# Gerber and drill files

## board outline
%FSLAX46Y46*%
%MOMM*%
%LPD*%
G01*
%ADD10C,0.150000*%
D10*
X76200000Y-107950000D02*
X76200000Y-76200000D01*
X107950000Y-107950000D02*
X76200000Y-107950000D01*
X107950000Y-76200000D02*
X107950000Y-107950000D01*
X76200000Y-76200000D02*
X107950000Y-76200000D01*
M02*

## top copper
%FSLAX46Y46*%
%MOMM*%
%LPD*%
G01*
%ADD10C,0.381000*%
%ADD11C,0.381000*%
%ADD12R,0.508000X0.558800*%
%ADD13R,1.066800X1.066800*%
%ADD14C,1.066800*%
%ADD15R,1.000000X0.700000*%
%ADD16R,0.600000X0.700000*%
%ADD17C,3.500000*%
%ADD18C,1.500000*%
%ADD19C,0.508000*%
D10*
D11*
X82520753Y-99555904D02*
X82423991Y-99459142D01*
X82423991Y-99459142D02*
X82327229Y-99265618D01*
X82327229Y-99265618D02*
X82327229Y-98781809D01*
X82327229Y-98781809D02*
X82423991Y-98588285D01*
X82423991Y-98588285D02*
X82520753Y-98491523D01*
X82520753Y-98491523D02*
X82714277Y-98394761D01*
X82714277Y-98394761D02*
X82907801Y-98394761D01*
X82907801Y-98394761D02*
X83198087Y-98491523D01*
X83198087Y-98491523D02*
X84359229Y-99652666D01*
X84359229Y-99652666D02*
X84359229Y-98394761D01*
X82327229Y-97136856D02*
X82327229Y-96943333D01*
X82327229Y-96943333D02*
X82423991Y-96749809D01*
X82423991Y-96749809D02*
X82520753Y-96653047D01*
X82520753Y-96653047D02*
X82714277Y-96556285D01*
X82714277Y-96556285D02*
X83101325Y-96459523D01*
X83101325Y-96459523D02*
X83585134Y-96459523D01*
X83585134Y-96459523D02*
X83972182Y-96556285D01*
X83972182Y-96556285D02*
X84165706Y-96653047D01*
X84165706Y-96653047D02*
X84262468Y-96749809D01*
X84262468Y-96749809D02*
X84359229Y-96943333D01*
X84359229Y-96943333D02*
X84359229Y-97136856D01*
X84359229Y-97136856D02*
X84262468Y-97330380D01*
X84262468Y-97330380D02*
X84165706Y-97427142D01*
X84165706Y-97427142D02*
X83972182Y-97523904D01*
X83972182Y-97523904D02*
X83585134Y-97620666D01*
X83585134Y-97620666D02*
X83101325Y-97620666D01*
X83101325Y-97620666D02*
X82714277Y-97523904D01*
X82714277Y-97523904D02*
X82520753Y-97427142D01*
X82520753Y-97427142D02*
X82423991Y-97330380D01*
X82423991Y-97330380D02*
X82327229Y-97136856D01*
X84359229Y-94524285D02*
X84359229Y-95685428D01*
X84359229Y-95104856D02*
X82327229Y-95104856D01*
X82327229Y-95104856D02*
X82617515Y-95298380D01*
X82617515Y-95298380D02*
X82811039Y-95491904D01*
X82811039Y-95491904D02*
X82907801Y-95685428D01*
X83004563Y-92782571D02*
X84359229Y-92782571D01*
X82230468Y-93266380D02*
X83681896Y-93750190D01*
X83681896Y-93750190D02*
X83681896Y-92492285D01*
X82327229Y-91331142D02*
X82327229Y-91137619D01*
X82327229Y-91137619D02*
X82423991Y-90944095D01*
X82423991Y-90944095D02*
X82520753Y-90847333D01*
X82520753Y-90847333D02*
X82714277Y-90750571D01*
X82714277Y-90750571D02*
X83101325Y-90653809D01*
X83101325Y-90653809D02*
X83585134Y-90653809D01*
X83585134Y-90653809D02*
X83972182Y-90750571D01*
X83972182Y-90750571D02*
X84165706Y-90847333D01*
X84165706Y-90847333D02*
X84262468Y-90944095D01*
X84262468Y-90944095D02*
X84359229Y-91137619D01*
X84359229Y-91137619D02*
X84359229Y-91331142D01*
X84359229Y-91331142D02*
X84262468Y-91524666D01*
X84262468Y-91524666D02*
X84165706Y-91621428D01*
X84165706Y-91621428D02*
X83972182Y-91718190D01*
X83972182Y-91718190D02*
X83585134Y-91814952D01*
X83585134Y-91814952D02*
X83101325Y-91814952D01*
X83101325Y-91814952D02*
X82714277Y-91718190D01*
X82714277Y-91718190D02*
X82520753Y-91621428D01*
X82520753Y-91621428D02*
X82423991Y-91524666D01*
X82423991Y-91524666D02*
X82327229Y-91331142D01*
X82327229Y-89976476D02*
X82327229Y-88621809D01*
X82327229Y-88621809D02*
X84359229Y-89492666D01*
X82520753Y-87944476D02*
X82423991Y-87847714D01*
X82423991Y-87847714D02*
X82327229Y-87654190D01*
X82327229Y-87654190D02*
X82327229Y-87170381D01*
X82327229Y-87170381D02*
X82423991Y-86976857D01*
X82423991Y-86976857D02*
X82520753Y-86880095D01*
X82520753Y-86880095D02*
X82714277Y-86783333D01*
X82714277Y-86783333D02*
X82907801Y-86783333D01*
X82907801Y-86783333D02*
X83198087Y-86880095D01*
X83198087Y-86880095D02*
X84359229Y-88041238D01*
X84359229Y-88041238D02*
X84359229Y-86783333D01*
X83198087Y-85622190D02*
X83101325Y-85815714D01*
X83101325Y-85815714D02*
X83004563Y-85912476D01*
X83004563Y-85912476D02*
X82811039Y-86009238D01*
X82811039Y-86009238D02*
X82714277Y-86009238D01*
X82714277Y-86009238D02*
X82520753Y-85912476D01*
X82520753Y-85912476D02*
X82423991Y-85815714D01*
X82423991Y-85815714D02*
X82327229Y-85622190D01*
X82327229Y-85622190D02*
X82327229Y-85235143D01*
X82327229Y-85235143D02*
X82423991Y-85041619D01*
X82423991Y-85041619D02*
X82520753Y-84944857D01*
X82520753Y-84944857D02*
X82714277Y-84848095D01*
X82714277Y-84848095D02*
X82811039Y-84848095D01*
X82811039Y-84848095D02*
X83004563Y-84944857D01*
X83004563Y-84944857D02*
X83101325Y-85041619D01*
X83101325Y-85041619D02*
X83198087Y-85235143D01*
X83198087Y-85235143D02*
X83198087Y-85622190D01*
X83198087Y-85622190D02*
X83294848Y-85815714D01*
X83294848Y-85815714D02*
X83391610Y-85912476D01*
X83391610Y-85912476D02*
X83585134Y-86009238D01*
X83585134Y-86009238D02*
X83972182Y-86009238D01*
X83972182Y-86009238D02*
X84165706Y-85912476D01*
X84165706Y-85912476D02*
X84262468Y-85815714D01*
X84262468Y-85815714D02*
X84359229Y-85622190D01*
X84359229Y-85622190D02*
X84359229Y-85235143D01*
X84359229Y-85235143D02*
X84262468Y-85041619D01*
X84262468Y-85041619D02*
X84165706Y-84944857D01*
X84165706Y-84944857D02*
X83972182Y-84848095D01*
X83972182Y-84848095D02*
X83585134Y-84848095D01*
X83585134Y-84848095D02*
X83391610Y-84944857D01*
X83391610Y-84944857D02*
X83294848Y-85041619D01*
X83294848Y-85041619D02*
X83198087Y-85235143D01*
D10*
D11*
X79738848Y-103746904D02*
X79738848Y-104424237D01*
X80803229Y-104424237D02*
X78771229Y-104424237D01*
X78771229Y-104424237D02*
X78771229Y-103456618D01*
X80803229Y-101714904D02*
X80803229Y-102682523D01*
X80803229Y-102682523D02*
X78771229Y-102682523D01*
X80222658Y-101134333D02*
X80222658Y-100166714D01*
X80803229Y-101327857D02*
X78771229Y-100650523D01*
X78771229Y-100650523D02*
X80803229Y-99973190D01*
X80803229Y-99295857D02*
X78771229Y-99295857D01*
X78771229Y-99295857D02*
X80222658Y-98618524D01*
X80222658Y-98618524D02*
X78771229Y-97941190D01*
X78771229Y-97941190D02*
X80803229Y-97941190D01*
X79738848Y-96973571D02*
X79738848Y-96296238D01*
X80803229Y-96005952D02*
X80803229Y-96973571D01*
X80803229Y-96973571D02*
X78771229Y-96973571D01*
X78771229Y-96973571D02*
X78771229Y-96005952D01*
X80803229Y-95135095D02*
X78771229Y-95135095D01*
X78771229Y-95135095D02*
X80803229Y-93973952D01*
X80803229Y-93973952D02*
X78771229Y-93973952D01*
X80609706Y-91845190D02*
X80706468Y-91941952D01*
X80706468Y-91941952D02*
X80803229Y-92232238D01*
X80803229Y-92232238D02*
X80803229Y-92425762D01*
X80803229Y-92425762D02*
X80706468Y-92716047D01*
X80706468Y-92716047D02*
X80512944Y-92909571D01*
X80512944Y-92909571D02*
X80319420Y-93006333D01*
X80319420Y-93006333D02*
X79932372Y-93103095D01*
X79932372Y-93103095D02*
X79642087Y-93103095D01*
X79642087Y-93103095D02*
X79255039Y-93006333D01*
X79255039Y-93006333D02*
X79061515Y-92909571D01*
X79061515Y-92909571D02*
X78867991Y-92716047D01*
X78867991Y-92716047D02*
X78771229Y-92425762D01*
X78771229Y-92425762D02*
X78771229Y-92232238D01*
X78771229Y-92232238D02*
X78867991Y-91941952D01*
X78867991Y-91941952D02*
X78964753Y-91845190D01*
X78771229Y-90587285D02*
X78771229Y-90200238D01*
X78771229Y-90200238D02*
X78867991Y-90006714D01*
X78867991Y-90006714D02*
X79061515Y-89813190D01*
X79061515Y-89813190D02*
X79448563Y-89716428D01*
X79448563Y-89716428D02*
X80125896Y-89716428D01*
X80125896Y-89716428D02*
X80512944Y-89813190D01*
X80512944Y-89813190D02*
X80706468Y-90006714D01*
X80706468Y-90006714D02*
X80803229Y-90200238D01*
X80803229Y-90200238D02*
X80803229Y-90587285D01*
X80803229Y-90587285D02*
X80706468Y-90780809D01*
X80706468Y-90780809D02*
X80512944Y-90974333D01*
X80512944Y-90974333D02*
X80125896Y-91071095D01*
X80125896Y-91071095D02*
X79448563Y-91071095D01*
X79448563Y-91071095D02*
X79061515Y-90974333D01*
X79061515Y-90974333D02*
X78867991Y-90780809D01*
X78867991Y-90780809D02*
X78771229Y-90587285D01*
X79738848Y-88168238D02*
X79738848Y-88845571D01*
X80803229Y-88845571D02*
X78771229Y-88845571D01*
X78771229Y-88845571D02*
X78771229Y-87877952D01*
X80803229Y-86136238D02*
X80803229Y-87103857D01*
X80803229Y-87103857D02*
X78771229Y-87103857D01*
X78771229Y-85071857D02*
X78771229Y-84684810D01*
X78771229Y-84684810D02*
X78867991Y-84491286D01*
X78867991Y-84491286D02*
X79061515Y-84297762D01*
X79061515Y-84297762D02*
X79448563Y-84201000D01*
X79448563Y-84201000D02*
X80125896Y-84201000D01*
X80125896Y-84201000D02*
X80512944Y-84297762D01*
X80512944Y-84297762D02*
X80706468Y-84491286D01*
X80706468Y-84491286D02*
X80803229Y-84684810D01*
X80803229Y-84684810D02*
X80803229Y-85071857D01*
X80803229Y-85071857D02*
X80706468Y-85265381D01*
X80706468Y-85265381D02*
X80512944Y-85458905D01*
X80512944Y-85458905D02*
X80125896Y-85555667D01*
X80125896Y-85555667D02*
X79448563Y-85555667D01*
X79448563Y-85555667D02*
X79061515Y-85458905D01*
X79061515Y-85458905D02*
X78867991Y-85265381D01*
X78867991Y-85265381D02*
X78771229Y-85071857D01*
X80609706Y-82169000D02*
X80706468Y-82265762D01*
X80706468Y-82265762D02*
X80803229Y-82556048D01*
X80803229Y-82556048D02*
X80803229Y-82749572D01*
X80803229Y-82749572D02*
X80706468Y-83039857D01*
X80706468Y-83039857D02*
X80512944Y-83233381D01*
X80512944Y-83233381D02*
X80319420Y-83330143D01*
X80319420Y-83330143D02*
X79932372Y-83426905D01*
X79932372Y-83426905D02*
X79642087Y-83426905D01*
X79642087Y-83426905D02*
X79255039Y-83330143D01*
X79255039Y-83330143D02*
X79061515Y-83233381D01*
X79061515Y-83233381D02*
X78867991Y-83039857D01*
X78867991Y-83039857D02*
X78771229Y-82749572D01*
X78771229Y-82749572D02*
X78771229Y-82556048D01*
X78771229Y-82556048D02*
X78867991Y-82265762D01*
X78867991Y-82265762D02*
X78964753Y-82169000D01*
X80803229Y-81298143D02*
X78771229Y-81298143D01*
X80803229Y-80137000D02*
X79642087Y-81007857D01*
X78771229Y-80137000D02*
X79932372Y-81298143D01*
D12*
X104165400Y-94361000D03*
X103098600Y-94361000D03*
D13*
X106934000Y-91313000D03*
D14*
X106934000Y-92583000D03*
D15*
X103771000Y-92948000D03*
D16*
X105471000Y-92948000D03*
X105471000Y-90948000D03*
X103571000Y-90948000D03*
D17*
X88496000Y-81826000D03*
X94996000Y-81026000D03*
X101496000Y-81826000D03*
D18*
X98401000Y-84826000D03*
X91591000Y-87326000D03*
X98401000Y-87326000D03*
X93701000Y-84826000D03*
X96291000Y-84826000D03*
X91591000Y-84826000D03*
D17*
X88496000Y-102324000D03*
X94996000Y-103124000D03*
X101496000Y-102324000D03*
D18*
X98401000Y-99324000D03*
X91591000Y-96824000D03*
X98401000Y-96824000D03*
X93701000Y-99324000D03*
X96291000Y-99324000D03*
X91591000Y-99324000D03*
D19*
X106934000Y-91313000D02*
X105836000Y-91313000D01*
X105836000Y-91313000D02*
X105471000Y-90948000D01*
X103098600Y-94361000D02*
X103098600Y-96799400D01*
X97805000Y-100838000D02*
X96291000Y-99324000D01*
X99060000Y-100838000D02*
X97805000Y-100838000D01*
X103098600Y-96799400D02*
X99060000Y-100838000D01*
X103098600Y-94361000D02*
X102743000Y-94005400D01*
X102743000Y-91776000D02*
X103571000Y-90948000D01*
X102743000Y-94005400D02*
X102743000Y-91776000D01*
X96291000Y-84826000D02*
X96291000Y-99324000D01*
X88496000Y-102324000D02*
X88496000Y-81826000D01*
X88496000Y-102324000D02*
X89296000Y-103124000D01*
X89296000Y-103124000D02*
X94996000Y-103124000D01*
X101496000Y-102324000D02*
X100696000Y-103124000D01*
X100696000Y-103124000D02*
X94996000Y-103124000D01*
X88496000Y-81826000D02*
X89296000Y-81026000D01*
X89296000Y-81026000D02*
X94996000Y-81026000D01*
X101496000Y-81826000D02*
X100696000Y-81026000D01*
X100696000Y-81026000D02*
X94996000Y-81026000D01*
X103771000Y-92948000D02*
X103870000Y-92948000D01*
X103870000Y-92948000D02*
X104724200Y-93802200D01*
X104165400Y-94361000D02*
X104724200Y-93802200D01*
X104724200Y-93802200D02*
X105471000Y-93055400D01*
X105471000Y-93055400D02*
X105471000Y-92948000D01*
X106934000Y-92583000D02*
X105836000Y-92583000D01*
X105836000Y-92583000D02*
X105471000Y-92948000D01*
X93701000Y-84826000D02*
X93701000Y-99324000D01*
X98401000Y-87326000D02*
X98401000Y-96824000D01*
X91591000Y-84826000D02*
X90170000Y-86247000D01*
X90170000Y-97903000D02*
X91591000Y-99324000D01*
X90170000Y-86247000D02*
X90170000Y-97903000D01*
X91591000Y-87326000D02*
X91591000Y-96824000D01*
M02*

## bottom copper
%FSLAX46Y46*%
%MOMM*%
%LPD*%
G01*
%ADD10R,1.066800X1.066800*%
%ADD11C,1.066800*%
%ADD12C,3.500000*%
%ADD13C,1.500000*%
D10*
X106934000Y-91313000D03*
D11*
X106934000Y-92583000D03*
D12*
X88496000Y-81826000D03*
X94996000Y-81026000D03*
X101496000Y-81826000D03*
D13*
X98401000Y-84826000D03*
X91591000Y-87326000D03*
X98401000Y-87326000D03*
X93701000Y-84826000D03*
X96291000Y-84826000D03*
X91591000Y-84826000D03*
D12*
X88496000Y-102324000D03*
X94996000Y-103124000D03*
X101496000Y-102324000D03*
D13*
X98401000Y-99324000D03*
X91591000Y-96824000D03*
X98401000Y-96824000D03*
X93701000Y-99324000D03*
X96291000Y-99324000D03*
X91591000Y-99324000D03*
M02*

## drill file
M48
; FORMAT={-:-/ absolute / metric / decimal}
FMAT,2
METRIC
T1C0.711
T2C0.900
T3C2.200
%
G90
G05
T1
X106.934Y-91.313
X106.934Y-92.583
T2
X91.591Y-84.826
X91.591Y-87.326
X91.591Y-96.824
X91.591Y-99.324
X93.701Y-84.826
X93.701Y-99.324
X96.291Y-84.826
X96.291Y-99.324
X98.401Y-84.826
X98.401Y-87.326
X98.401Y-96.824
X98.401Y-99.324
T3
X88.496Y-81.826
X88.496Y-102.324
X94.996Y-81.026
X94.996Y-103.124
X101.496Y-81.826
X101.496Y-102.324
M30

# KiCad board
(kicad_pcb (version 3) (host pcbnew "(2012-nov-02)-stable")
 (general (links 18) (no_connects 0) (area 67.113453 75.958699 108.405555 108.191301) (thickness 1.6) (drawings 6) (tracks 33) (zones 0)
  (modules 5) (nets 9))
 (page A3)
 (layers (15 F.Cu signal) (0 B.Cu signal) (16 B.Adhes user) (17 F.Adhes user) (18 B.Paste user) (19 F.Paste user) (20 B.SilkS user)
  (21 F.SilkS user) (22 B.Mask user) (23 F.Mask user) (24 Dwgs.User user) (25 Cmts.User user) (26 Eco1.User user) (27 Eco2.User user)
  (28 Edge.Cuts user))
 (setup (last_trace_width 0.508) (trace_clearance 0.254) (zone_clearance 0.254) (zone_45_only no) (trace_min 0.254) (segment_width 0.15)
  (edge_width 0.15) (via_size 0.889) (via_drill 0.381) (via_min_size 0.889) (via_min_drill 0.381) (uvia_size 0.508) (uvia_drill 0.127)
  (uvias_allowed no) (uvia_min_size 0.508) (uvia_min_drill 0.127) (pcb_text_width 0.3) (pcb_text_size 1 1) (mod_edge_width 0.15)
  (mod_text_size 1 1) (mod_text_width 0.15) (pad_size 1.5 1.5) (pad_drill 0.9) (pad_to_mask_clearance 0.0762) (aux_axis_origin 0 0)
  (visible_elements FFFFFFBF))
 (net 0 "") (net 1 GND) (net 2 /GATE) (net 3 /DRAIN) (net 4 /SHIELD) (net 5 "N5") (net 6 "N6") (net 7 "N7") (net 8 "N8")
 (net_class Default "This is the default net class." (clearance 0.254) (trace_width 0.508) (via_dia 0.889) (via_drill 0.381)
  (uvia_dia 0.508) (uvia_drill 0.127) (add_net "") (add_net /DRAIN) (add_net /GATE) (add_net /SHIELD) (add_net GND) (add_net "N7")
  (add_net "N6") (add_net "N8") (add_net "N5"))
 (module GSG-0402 (layer F.Cu) (at 103.632 94.361) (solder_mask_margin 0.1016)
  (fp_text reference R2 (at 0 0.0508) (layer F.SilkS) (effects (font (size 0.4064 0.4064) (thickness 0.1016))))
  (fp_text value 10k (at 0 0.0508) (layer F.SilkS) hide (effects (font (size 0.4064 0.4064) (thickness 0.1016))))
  (pad 2 smd rect (at 0.5334 0) (size 0.508 0.5588) (layers F.Cu F.Paste F.Mask) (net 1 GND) (solder_mask_margin 0.1016))
  (pad 1 smd rect (at -0.5334 0) (size 0.508 0.5588) (layers F.Cu F.Paste F.Mask) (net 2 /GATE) (die_length -2147.483648)
   (solder_mask_margin 0.1016)))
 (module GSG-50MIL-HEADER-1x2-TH (layer F.Cu) (at 106.934 91.948 270)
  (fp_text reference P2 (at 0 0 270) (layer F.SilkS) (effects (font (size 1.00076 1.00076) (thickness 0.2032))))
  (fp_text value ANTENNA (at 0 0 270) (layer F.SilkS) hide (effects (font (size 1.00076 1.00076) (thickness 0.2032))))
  (pad 1 thru_hole rect (at -0.635 0 270) (size 1.0668 1.0668) (drill 0.7112) (layers *.Cu *.Mask) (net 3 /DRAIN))
  (pad 2 thru_hole circle (at 0.635 0 270) (size 1.0668 1.0668) (drill 0.7112) (layers *.Cu *.Mask) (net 1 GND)))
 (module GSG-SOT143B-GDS (layer F.Cu) (at 104.521 91.948)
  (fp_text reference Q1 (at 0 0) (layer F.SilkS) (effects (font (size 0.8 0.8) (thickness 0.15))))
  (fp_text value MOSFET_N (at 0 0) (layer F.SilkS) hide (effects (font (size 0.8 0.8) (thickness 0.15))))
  (pad B smd rect (at -0.75 1) (size 1 0.7) (layers F.Cu F.Paste F.Mask) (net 1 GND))
  (pad S smd rect (at 0.95 1) (size 0.6 0.7) (layers F.Cu F.Paste F.Mask) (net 1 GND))
  (pad D smd rect (at 0.95 -1) (size 0.6 0.7) (layers F.Cu F.Paste F.Mask) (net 3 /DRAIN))
  (pad G smd rect (at -0.95 -1) (size 0.6 0.7) (layers F.Cu F.Paste F.Mask) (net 2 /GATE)))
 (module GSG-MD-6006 (layer B.Cu) (at 94.996 81.026 180)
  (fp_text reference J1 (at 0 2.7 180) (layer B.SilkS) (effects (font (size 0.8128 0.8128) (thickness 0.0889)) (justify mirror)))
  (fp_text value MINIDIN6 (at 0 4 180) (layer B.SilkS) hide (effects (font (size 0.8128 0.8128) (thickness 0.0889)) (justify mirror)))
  (pad 0 thru_hole circle (at 6.5 -0.8 180) (size 3.5 3.5) (drill 2.2) (layers *.Cu *.Mask B.SilkS) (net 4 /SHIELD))
  (pad 0 thru_hole circle (at 0 0 180) (size 3.5 3.5) (drill 2.2) (layers *.Cu *.Mask B.SilkS) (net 4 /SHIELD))
  (pad 0 thru_hole circle (at -6.5 -0.8 180) (size 3.5 3.5) (drill 2.2) (layers *.Cu *.Mask B.SilkS) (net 4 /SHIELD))
  (pad 3 thru_hole circle (at -3.405 -3.8 180) (size 1.5 1.5) (drill 0.9) (layers *.Cu *.Mask B.SilkS))
  (pad 6 thru_hole circle (at 3.405 -6.3 180) (size 1.5 1.5) (drill 0.9) (layers *.Cu *.Mask B.SilkS) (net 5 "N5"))
  (pad 5 thru_hole circle (at -3.405 -6.3 180) (size 1.5 1.5) (drill 0.9) (layers *.Cu *.Mask B.SilkS) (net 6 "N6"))
  (pad 2 thru_hole circle (at 1.295 -3.8 180) (size 1.5 1.5) (drill 0.9) (layers *.Cu *.Mask B.SilkS) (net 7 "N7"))
  (pad 1 thru_hole circle (at -1.295 -3.8 180) (size 1.5 1.5) (drill 0.9) (layers *.Cu *.Mask B.SilkS) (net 2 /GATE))
  (pad 4 thru_hole circle (at 3.405 -3.8 180) (size 1.5 1.5) (drill 0.9) (layers *.Cu *.Mask B.SilkS) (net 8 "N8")))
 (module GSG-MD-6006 (layer F.Cu) (at 94.996 103.124 180)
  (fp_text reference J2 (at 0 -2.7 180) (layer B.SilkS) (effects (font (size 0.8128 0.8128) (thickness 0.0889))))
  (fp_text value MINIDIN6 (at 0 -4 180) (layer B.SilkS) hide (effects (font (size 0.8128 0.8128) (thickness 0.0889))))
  (pad 0 thru_hole circle (at 6.5 0.8 180) (size 3.5 3.5) (drill 2.2) (layers *.Cu *.Mask F.SilkS) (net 4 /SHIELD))
  (pad 0 thru_hole circle (at 0 0 180) (size 3.5 3.5) (drill 2.2) (layers *.Cu *.Mask F.SilkS) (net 4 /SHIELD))
  (pad 0 thru_hole circle (at -6.5 0.8 180) (size 3.5 3.5) (drill 2.2) (layers *.Cu *.Mask F.SilkS) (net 4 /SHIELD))
  (pad 3 thru_hole circle (at -3.405 3.8 180) (size 1.5 1.5) (drill 0.9) (layers *.Cu *.Mask F.SilkS))
  (pad 6 thru_hole circle (at 3.405 6.3 180) (size 1.5 1.5) (drill 0.9) (layers *.Cu *.Mask F.SilkS) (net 5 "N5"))
  (pad 5 thru_hole circle (at -3.405 6.3 180) (size 1.5 1.5) (drill 0.9) (layers *.Cu *.Mask F.SilkS) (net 6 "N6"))
  (pad 2 thru_hole circle (at 1.295 3.8 180) (size 1.5 1.5) (drill 0.9) (layers *.Cu *.Mask F.SilkS) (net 7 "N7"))
  (pad 1 thru_hole circle (at -1.295 3.8 180) (size 1.5 1.5) (drill 0.9) (layers *.Cu *.Mask F.SilkS) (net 2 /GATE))
  (pad 4 thru_hole circle (at 3.405 3.8 180) (size 1.5 1.5) (drill 0.9) (layers *.Cu *.Mask F.SilkS) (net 8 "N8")))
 (gr_line (start 76.2 107.95) (end 76.2 76.2) (angle 90) (layer Edge.Cuts) (width 0.15))
 (gr_line (start 107.95 107.95) (end 76.2 107.95) (angle 90) (layer Edge.Cuts) (width 0.15))
 (gr_line (start 107.95 76.2) (end 107.95 107.95) (angle 90) (layer Edge.Cuts) (width 0.15))
 (gr_line (start 76.2 76.2) (end 107.95 76.2) (angle 90) (layer Edge.Cuts) (width 0.15))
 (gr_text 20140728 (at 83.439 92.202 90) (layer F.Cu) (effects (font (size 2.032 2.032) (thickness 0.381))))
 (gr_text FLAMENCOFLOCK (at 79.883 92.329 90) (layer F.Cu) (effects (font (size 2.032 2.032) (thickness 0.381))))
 (segment (start 106.934 91.313) (end 105.836 91.313) (width 0.508) (layer F.Cu) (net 3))
 (segment (start 105.836 91.313) (end 105.471 90.948) (width 0.508) (layer F.Cu) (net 3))
 (segment (start 103.0986 94.361) (end 103.0986 96.7994) (width 0.508) (layer F.Cu) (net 2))
 (segment (start 97.805 100.838) (end 96.291 99.324) (width 0.508) (layer F.Cu) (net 2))
 (segment (start 99.06 100.838) (end 97.805 100.838) (width 0.508) (layer F.Cu) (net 2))
 (segment (start 103.0986 96.7994) (end 99.06 100.838) (width 0.508) (layer F.Cu) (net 2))
 (segment (start 103.0986 94.361) (end 102.743 94.0054) (width 0.508) (layer F.Cu) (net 2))
 (segment (start 102.743 91.776) (end 103.571 90.948) (width 0.508) (layer F.Cu) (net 2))
 (segment (start 102.743 94.0054) (end 102.743 91.776) (width 0.508) (layer F.Cu) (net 2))
 (segment (start 96.291 84.826) (end 96.291 99.324) (width 0.508) (layer F.Cu) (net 2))
 (segment (start 88.496 102.324) (end 88.496 81.826) (width 0.508) (layer F.Cu) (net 4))
 (segment (start 88.496 102.324) (end 89.296 103.124) (width 0.508) (layer F.Cu) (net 4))
 (segment (start 89.296 103.124) (end 94.996 103.124) (width 0.508) (layer F.Cu) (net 4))
 (segment (start 101.496 102.324) (end 100.696 103.124) (width 0.508) (layer F.Cu) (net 4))
 (segment (start 100.696 103.124) (end 94.996 103.124) (width 0.508) (layer F.Cu) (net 4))
 (segment (start 88.496 81.826) (end 89.296 81.026) (width 0.508) (layer F.Cu) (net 4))
 (segment (start 89.296 81.026) (end 94.996 81.026) (width 0.508) (layer F.Cu) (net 4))
 (segment (start 101.496 81.826) (end 100.696 81.026) (width 0.508) (layer F.Cu) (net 4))
 (segment (start 100.696 81.026) (end 94.996 81.026) (width 0.508) (layer F.Cu) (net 4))
 (segment (start 103.771 92.948) (end 103.87 92.948) (width 0.508) (layer F.Cu) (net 1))
 (segment (start 103.87 92.948) (end 104.7242 93.8022) (width 0.508) (layer F.Cu) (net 1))
 (segment (start 104.1654 94.361) (end 104.7242 93.8022) (width 0.508) (layer F.Cu) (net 1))
 (segment (start 104.7242 93.8022) (end 105.471 93.0554) (width 0.508) (layer F.Cu) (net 1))
 (segment (start 105.471 93.0554) (end 105.471 92.948) (width 0.508) (layer F.Cu) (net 1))
 (segment (start 106.934 92.583) (end 105.836 92.583) (width 0.508) (layer F.Cu) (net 1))
 (segment (start 105.836 92.583) (end 105.471 92.948) (width 0.508) (layer F.Cu) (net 1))
 (segment (start 93.701 84.826) (end 93.701 99.324) (width 0.508) (layer F.Cu) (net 7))
 (segment (start 98.401 87.326) (end 98.401 96.824) (width 0.508) (layer F.Cu) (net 6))
 (segment (start 91.591 84.826) (end 90.17 86.247) (width 0.508) (layer F.Cu) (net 8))
 (segment (start 90.17 97.903) (end 91.591 99.324) (width 0.508) (layer F.Cu) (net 8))
 (segment (start 90.17 86.247) (end 90.17 97.903) (width 0.508) (layer F.Cu) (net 8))
 (segment (start 91.591 87.326) (end 91.591 96.824) (width 0.508) (layer F.Cu) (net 5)))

